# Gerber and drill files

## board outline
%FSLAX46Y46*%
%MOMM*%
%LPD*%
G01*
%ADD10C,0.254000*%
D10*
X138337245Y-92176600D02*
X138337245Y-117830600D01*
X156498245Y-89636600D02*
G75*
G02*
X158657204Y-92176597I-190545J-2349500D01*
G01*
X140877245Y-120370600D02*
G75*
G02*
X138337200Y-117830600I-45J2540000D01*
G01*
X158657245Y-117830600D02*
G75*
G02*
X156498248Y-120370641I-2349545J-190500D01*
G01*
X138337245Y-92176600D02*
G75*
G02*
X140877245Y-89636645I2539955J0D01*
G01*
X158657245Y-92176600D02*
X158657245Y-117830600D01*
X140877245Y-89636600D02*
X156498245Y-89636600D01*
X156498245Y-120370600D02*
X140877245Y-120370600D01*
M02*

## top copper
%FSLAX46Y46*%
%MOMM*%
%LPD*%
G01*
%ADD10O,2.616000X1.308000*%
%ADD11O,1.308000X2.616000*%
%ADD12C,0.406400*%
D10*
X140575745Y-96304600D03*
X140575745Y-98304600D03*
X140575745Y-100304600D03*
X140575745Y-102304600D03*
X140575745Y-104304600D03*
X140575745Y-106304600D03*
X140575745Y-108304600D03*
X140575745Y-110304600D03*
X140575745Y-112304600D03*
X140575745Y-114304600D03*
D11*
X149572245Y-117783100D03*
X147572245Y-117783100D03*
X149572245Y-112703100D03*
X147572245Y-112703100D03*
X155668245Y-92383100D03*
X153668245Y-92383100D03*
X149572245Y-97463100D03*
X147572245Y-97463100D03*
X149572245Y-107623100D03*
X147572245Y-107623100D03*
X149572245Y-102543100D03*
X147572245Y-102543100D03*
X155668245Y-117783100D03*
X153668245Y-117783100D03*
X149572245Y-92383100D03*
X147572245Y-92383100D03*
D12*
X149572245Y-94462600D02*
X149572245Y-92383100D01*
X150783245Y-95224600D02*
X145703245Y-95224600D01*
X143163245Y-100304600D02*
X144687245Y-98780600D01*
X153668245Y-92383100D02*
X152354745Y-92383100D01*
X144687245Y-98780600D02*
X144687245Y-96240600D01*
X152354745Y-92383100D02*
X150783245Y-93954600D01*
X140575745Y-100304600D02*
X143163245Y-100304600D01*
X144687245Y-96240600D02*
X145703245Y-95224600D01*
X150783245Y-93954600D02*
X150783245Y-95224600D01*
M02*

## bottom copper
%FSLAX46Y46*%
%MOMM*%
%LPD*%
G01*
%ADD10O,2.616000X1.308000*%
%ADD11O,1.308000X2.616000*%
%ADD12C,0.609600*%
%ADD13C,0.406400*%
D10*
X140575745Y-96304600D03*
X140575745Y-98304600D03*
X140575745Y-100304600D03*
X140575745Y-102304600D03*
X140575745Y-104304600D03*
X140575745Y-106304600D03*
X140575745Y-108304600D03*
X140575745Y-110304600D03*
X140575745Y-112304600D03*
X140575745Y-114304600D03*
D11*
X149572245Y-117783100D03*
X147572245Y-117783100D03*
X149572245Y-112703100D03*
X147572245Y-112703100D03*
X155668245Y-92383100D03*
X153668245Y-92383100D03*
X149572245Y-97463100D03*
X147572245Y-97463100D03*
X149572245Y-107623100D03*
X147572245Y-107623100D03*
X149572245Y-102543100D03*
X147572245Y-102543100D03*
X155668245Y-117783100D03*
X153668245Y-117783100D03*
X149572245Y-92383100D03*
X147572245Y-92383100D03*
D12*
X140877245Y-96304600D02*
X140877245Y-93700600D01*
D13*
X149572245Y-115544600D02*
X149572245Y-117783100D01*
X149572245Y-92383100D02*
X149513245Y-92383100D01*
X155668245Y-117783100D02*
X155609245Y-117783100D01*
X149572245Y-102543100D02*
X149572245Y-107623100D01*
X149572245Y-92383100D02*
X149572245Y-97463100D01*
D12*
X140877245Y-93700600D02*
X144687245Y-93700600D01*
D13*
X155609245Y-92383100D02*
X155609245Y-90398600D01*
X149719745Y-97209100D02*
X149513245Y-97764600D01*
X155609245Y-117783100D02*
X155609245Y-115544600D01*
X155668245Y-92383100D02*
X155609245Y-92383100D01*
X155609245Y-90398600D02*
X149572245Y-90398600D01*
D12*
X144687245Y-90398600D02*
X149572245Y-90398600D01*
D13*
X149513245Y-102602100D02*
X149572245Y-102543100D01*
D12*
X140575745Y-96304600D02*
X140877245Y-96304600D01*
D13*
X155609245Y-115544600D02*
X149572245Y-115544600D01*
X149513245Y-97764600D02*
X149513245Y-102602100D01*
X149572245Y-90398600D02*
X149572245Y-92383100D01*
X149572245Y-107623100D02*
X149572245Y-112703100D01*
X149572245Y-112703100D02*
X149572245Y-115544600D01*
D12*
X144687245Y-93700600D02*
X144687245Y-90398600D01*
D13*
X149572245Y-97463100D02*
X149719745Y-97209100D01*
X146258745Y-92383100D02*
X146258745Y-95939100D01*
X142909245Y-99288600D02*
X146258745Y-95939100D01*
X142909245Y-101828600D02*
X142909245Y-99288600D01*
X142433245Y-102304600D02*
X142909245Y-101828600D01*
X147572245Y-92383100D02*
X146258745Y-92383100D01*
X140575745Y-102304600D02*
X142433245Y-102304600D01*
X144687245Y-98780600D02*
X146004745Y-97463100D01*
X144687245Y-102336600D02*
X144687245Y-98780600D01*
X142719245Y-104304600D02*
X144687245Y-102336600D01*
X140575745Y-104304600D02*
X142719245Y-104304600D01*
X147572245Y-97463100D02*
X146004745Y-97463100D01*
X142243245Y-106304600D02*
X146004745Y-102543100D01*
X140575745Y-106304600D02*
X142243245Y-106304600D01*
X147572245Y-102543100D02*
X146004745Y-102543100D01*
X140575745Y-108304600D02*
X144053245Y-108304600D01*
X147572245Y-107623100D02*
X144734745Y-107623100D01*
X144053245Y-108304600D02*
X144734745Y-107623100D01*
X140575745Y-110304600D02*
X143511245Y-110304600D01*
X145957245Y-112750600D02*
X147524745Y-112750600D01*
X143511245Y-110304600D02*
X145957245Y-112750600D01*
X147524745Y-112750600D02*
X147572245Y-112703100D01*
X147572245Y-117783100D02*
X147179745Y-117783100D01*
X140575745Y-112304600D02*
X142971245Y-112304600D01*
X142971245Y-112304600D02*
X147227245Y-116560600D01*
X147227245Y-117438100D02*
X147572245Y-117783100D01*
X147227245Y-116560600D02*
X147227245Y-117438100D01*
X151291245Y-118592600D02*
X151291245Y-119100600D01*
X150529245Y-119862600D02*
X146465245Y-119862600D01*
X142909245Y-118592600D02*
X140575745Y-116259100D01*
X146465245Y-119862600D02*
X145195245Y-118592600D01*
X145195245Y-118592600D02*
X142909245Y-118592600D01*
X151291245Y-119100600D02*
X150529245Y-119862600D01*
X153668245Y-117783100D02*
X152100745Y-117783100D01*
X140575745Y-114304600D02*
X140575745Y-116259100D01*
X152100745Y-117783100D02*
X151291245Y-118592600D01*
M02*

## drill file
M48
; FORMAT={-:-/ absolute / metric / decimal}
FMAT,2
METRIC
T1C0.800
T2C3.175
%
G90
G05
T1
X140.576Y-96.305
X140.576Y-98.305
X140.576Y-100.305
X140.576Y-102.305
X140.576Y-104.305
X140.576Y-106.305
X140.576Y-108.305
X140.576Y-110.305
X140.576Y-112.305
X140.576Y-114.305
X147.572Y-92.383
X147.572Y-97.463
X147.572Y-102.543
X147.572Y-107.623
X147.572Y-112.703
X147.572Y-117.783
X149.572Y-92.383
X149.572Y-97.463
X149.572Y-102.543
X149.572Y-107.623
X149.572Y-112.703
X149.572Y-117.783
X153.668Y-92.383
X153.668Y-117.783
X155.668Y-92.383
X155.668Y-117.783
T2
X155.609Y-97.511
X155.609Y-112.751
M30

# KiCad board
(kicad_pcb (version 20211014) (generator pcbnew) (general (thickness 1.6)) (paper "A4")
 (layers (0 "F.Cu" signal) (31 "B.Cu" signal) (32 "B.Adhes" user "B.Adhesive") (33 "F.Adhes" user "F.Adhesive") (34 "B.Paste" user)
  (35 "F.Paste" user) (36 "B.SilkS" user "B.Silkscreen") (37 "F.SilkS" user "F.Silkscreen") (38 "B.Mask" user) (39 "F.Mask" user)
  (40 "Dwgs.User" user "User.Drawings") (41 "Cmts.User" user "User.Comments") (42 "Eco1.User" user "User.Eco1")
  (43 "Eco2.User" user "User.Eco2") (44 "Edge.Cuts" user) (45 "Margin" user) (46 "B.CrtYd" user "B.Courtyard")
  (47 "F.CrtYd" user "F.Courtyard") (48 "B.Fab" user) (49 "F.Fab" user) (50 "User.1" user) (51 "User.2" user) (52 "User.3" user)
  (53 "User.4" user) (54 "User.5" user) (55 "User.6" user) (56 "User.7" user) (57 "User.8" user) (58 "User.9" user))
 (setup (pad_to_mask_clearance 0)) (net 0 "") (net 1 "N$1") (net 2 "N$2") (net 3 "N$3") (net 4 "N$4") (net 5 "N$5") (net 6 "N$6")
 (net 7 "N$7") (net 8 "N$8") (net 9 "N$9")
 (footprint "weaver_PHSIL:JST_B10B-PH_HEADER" (layer "F.Cu") (at 140.623245 100.3046 90)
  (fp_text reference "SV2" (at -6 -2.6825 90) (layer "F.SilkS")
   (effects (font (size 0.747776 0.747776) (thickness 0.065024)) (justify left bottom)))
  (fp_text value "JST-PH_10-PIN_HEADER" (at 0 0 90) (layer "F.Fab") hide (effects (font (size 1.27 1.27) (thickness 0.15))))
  (pad "P1" thru_hole oval (at 4 -0.0475 180) (size 2.616 1.308) (drill 0.8) (layers *.Cu *.Mask) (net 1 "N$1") (solder_mask_margin 0.1016))
  (pad "P2" thru_hole oval (at 2 -0.0475 180) (size 2.616 1.308) (drill 0.8) (layers *.Cu *.Mask) (solder_mask_margin 0.1016))
  (pad "P3" thru_hole oval (at 0 -0.0475 180) (size 2.616 1.308) (drill 0.8) (layers *.Cu *.Mask) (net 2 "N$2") (solder_mask_margin 0.1016))
  (pad "P4" thru_hole oval (at -2 -0.0475 180) (size 2.616 1.308) (drill 0.8) (layers *.Cu *.Mask) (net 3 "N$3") (solder_mask_margin 0.1016))
  (pad "P5" thru_hole oval (at -4 -0.0475 180) (size 2.616 1.308) (drill 0.8) (layers *.Cu *.Mask) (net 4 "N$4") (solder_mask_margin 0.1016))
  (pad "P6" thru_hole oval (at -6 -0.0475 180) (size 2.616 1.308) (drill 0.8) (layers *.Cu *.Mask) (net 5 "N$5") (solder_mask_margin 0.1016))
  (pad "P7" thru_hole oval (at -8 -0.0475 180) (size 2.616 1.308) (drill 0.8) (layers *.Cu *.Mask) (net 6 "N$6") (solder_mask_margin 0.1016))
  (pad "P8" thru_hole oval (at -10 -0.0475 180) (size 2.616 1.308) (drill 0.8) (layers *.Cu *.Mask) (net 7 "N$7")
   (solder_mask_margin 0.1016))
  (pad "P9" thru_hole oval (at -12 -0.0475 180) (size 2.616 1.308) (drill 0.8) (layers *.Cu *.Mask) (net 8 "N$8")
   (solder_mask_margin 0.1016))
  (pad "P10" thru_hole oval (at -14 -0.0475 180) (size 2.616 1.308) (drill 0.8) (layers *.Cu *.Mask) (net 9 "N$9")
   (solder_mask_margin 0.1016)))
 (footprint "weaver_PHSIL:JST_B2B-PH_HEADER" (layer "F.Cu") (at 148.497245 117.8306)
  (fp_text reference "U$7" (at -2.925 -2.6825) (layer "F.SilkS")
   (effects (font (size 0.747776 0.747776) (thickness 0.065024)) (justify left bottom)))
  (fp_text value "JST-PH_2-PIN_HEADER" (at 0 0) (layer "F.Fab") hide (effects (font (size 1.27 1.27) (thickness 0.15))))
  (pad "P1" thru_hole oval (at 1.075 -0.0475 90) (size 2.616 1.308) (drill 0.8) (layers *.Cu *.Mask) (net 1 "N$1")
   (solder_mask_margin 0.1016))
  (pad "P2" thru_hole oval (at -0.925 -0.0475 90) (size 2.616 1.308) (drill 0.8) (layers *.Cu *.Mask) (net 8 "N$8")
   (solder_mask_margin 0.1016)))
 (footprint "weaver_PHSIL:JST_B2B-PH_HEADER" (layer "F.Cu") (at 148.497245 112.7506)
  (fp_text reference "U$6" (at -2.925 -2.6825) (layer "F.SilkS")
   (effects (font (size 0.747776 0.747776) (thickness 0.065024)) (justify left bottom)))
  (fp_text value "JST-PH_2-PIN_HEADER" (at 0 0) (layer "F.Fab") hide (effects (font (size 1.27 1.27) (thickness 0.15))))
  (pad "P1" thru_hole oval (at 1.075 -0.0475 90) (size 2.616 1.308) (drill 0.8) (layers *.Cu *.Mask) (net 1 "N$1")
   (solder_mask_margin 0.1016))
  (pad "P2" thru_hole oval (at -0.925 -0.0475 90) (size 2.616 1.308) (drill 0.8) (layers *.Cu *.Mask) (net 7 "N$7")
   (solder_mask_margin 0.1016)))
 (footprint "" (layer "F.Cu") (at 155.609245 112.7506)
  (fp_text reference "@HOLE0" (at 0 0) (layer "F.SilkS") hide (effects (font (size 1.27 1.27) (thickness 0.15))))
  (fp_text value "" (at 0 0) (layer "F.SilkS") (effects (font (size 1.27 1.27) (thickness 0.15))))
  (pad "" np_thru_hole circle (at 0 0) (size 3.175 3.175) (drill 3.175) (layers *.Cu *.Mask)))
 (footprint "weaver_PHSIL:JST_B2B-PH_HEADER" (layer "F.Cu") (at 154.593245 92.4306)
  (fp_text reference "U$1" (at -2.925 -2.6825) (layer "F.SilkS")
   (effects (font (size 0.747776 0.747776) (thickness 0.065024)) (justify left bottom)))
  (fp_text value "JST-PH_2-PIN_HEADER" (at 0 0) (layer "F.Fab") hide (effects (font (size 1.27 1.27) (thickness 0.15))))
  (pad "P1" thru_hole oval (at 1.075 -0.0475 90) (size 2.616 1.308) (drill 0.8) (layers *.Cu *.Mask) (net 1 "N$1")
   (solder_mask_margin 0.1016))
  (pad "P2" thru_hole oval (at -0.925 -0.0475 90) (size 2.616 1.308) (drill 0.8) (layers *.Cu *.Mask) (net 2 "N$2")
   (solder_mask_margin 0.1016)))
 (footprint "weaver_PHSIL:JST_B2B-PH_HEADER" (layer "F.Cu") (at 148.497245 97.5106)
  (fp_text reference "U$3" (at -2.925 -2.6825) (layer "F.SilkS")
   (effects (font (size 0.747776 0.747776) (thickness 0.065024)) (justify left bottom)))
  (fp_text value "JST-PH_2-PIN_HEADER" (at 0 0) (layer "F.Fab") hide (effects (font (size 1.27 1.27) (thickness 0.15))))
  (pad "P1" thru_hole oval (at 1.075 -0.0475 90) (size 2.616 1.308) (drill 0.8) (layers *.Cu *.Mask) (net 1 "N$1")
   (solder_mask_margin 0.1016))
  (pad "P2" thru_hole oval (at -0.925 -0.0475 90) (size 2.616 1.308) (drill 0.8) (layers *.Cu *.Mask) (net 4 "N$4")
   (solder_mask_margin 0.1016)))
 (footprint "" (layer "F.Cu") (at 155.609245 97.5106)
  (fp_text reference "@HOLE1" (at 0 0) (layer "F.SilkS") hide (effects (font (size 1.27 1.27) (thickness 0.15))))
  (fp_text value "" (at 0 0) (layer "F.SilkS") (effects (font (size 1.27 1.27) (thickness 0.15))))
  (pad "" np_thru_hole circle (at 0 0) (size 3.175 3.175) (drill 3.175) (layers *.Cu *.Mask)))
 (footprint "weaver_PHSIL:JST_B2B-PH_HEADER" (layer "F.Cu") (at 148.497245 107.6706)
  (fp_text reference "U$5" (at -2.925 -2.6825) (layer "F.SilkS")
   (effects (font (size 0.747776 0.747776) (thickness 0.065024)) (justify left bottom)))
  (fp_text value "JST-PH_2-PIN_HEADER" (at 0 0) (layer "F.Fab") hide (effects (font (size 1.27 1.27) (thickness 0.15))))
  (pad "P1" thru_hole oval (at 1.075 -0.0475 90) (size 2.616 1.308) (drill 0.8) (layers *.Cu *.Mask) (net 1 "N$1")
   (solder_mask_margin 0.1016))
  (pad "P2" thru_hole oval (at -0.925 -0.0475 90) (size 2.616 1.308) (drill 0.8) (layers *.Cu *.Mask) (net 6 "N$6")
   (solder_mask_margin 0.1016)))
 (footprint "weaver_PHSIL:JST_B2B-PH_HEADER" (layer "F.Cu") (at 148.497245 102.5906)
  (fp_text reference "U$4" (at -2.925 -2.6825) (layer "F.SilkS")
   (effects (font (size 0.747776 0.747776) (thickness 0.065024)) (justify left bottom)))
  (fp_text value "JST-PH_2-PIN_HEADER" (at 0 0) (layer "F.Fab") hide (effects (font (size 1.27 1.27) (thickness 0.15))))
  (pad "P1" thru_hole oval (at 1.075 -0.0475 90) (size 2.616 1.308) (drill 0.8) (layers *.Cu *.Mask) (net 1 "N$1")
   (solder_mask_margin 0.1016))
  (pad "P2" thru_hole oval (at -0.925 -0.0475 90) (size 2.616 1.308) (drill 0.8) (layers *.Cu *.Mask) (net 5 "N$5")
   (solder_mask_margin 0.1016)))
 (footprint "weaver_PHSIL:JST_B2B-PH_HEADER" (layer "F.Cu") (at 154.593245 117.8306)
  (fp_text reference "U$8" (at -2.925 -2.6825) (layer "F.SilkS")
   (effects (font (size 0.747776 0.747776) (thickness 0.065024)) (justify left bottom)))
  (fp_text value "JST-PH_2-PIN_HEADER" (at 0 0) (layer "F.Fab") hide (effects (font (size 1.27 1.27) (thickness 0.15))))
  (pad "P1" thru_hole oval (at 1.075 -0.0475 90) (size 2.616 1.308) (drill 0.8) (layers *.Cu *.Mask) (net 1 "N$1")
   (solder_mask_margin 0.1016))
  (pad "P2" thru_hole oval (at -0.925 -0.0475 90) (size 2.616 1.308) (drill 0.8) (layers *.Cu *.Mask) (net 9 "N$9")
   (solder_mask_margin 0.1016)))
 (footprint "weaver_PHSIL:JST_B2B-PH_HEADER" (layer "F.Cu") (at 148.497245 92.4306)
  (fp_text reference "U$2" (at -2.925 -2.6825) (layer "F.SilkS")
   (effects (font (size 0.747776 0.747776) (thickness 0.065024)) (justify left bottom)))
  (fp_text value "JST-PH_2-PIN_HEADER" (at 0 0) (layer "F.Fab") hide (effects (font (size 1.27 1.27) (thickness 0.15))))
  (pad "P1" thru_hole oval (at 1.075 -0.0475 90) (size 2.616 1.308) (drill 0.8) (layers *.Cu *.Mask) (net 1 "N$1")
   (solder_mask_margin 0.1016))
  (pad "P2" thru_hole oval (at -0.925 -0.0475 90) (size 2.616 1.308) (drill 0.8) (layers *.Cu *.Mask) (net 3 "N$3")
   (solder_mask_margin 0.1016)))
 (gr_line (start 138.337245 92.1766) (end 138.337245 117.8306) (layer "Edge.Cuts") (width 0.254))
 (gr_arc (start 156.498245 89.6366) (mid 158.103796 90.459456) (end 158.657245 92.1766) (layer "Edge.Cuts") (width 0.254))
 (gr_arc (start 140.877245 120.3706) (mid 139.081194 119.626651) (end 138.337245 117.8306) (layer "Edge.Cuts") (width 0.254))
 (gr_arc (start 158.657245 117.8306) (mid 158.103796 119.547744) (end 156.498245 120.3706) (layer "Edge.Cuts") (width 0.254))
 (gr_arc (start 138.337245 92.1766) (mid 139.081194 90.380549) (end 140.877245 89.6366) (layer "Edge.Cuts") (width 0.254))
 (gr_line (start 158.657245 92.1766) (end 158.657245 117.8306) (layer "Edge.Cuts") (width 0.254))
 (gr_line (start 140.877245 89.6366) (end 156.498245 89.6366) (layer "Edge.Cuts") (width 0.254))
 (gr_line (start 156.498245 120.3706) (end 140.877245 120.3706) (layer "Edge.Cuts") (width 0.254))
 (segment (start 149.572245 94.4626) (end 149.572245 92.3831) (width 0.4064) (layer "F.Cu") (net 1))
 (segment (start 140.877245 96.3046) (end 140.877245 93.7006) (width 0.6096) (layer "B.Cu") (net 1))
 (segment (start 149.572245 115.5446) (end 149.572245 117.7831) (width 0.4064) (layer "B.Cu") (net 1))
 (segment (start 149.572245 92.3831) (end 149.513245 92.3831) (width 0.4064) (layer "B.Cu") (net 1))
 (segment (start 155.668245 117.7831) (end 155.609245 117.7831) (width 0.4064) (layer "B.Cu") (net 1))
 (segment (start 149.572245 102.5431) (end 149.572245 107.6231) (width 0.4064) (layer "B.Cu") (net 1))
 (segment (start 149.572245 92.3831) (end 149.572245 97.4631) (width 0.4064) (layer "B.Cu") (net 1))
 (segment (start 140.877245 93.7006) (end 144.687245 93.7006) (width 0.6096) (layer "B.Cu") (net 1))
 (segment (start 155.609245 92.3831) (end 155.609245 90.3986) (width 0.4064) (layer "B.Cu") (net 1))
 (segment (start 149.719745 97.2091) (end 149.513245 97.7646) (width 0.4064) (layer "B.Cu") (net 1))
 (segment (start 155.609245 117.7831) (end 155.609245 115.5446) (width 0.4064) (layer "B.Cu") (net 1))
 (segment (start 155.668245 92.3831) (end 155.609245 92.3831) (width 0.4064) (layer "B.Cu") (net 1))
 (segment (start 155.609245 90.3986) (end 149.572245 90.3986) (width 0.4064) (layer "B.Cu") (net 1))
 (segment (start 144.687245 90.3986) (end 149.572245 90.3986) (width 0.6096) (layer "B.Cu") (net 1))
 (segment (start 149.513245 102.6021) (end 149.572245 102.5431) (width 0.4064) (layer "B.Cu") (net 1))
 (segment (start 140.575745 96.3046) (end 140.877245 96.3046) (width 0.6096) (layer "B.Cu") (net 1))
 (segment (start 155.609245 115.5446) (end 149.572245 115.5446) (width 0.4064) (layer "B.Cu") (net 1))
 (segment (start 149.513245 97.7646) (end 149.513245 102.6021) (width 0.4064) (layer "B.Cu") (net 1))
 (segment (start 149.572245 90.3986) (end 149.572245 92.3831) (width 0.4064) (layer "B.Cu") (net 1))
 (segment (start 149.572245 107.6231) (end 149.572245 112.7031) (width 0.4064) (layer "B.Cu") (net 1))
 (segment (start 149.572245 112.7031) (end 149.572245 115.5446) (width 0.4064) (layer "B.Cu") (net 1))
 (segment (start 144.687245 93.7006) (end 144.687245 90.3986) (width 0.6096) (layer "B.Cu") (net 1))
 (segment (start 149.572245 97.4631) (end 149.719745 97.2091) (width 0.4064) (layer "B.Cu") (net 1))
 (segment (start 146.258745 92.3831) (end 146.258745 95.9391) (width 0.4064) (layer "B.Cu") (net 3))
 (segment (start 142.909245 99.2886) (end 146.258745 95.9391) (width 0.4064) (layer "B.Cu") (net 3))
 (segment (start 142.909245 101.8286) (end 142.909245 99.2886) (width 0.4064) (layer "B.Cu") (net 3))
 (segment (start 142.433245 102.3046) (end 142.909245 101.8286) (width 0.4064) (layer "B.Cu") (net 3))
 (segment (start 147.572245 92.3831) (end 146.258745 92.3831) (width 0.4064) (layer "B.Cu") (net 3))
 (segment (start 140.575745 102.3046) (end 142.433245 102.3046) (width 0.4064) (layer "B.Cu") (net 3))
 (segment (start 144.687245 98.7806) (end 146.004745 97.4631) (width 0.4064) (layer "B.Cu") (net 4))
 (segment (start 144.687245 102.3366) (end 144.687245 98.7806) (width 0.4064) (layer "B.Cu") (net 4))
 (segment (start 142.719245 104.3046) (end 144.687245 102.3366) (width 0.4064) (layer "B.Cu") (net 4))
 (segment (start 140.575745 104.3046) (end 142.719245 104.3046) (width 0.4064) (layer "B.Cu") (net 4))
 (segment (start 147.572245 97.4631) (end 146.004745 97.4631) (width 0.4064) (layer "B.Cu") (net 4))
 (segment (start 142.243245 106.3046) (end 146.004745 102.5431) (width 0.4064) (layer "B.Cu") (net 5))
 (segment (start 140.575745 106.3046) (end 142.243245 106.3046) (width 0.4064) (layer "B.Cu") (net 5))
 (segment (start 147.572245 102.5431) (end 146.004745 102.5431) (width 0.4064) (layer "B.Cu") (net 5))
 (segment (start 140.575745 108.3046) (end 144.053245 108.3046) (width 0.4064) (layer "B.Cu") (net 6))
 (segment (start 147.572245 107.6231) (end 144.734745 107.6231) (width 0.4064) (layer "B.Cu") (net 6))
 (segment (start 144.053245 108.3046) (end 144.734745 107.6231) (width 0.4064) (layer "B.Cu") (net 6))
 (segment (start 140.575745 110.3046) (end 143.511245 110.3046) (width 0.4064) (layer "B.Cu") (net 7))
 (segment (start 145.957245 112.7506) (end 147.524745 112.7506) (width 0.4064) (layer "B.Cu") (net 7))
 (segment (start 143.511245 110.3046) (end 145.957245 112.7506) (width 0.4064) (layer "B.Cu") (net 7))
 (segment (start 147.524745 112.7506) (end 147.572245 112.7031) (width 0.4064) (layer "B.Cu") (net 7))
 (segment (start 147.572245 117.7831) (end 147.179745 117.7831) (width 0.4064) (layer "B.Cu") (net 8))
 (segment (start 140.575745 112.3046) (end 142.971245 112.3046) (width 0.4064) (layer "B.Cu") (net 8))
 (segment (start 142.971245 112.3046) (end 147.227245 116.5606) (width 0.4064) (layer "B.Cu") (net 8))
 (segment (start 147.227245 117.4381) (end 147.572245 117.7831) (width 0.4064) (layer "B.Cu") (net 8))
 (segment (start 147.227245 116.5606) (end 147.227245 117.4381) (width 0.4064) (layer "B.Cu") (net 8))
 (segment (start 151.291245 118.5926) (end 151.291245 119.1006) (width 0.4064) (layer "B.Cu") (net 9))
 (segment (start 150.529245 119.8626) (end 146.465245 119.8626) (width 0.4064) (layer "B.Cu") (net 9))
 (segment (start 142.909245 118.5926) (end 140.575745 116.2591) (width 0.4064) (layer "B.Cu") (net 9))
 (segment (start 146.465245 119.8626) (end 145.195245 118.5926) (width 0.4064) (layer "B.Cu") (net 9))
 (segment (start 145.195245 118.5926) (end 142.909245 118.5926) (width 0.4064) (layer "B.Cu") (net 9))
 (segment (start 151.291245 119.1006) (end 150.529245 119.8626) (width 0.4064) (layer "B.Cu") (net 9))
 (segment (start 153.668245 117.7831) (end 152.100745 117.7831) (width 0.4064) (layer "B.Cu") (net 9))
 (segment (start 140.575745 114.3046) (end 140.575745 116.2591) (width 0.4064) (layer "B.Cu") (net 9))
 (segment (start 152.100745 117.7831) (end 151.291245 118.5926) (width 0.4064) (layer "B.Cu") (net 9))
 (segment (start 150.783245 95.2246) (end 145.703245 95.2246) (width 0.4064) (layer "F.Cu") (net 2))
 (segment (start 143.163245 100.3046) (end 144.687245 98.7806) (width 0.4064) (layer "F.Cu") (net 2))
 (segment (start 153.668245 92.3831) (end 152.354745 92.3831) (width 0.4064) (layer "F.Cu") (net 2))
 (segment (start 144.687245 98.7806) (end 144.687245 96.2406) (width 0.4064) (layer "F.Cu") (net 2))
 (segment (start 152.354745 92.3831) (end 150.783245 93.9546) (width 0.4064) (layer "F.Cu") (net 2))
 (segment (start 140.575745 100.3046) (end 143.163245 100.3046) (width 0.4064) (layer "F.Cu") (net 2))
 (segment (start 144.687245 96.2406) (end 145.703245 95.2246) (width 0.4064) (layer "F.Cu") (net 2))
 (segment (start 150.783245 93.9546) (end 150.783245 95.2246) (width 0.4064) (layer "F.Cu") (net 2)))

